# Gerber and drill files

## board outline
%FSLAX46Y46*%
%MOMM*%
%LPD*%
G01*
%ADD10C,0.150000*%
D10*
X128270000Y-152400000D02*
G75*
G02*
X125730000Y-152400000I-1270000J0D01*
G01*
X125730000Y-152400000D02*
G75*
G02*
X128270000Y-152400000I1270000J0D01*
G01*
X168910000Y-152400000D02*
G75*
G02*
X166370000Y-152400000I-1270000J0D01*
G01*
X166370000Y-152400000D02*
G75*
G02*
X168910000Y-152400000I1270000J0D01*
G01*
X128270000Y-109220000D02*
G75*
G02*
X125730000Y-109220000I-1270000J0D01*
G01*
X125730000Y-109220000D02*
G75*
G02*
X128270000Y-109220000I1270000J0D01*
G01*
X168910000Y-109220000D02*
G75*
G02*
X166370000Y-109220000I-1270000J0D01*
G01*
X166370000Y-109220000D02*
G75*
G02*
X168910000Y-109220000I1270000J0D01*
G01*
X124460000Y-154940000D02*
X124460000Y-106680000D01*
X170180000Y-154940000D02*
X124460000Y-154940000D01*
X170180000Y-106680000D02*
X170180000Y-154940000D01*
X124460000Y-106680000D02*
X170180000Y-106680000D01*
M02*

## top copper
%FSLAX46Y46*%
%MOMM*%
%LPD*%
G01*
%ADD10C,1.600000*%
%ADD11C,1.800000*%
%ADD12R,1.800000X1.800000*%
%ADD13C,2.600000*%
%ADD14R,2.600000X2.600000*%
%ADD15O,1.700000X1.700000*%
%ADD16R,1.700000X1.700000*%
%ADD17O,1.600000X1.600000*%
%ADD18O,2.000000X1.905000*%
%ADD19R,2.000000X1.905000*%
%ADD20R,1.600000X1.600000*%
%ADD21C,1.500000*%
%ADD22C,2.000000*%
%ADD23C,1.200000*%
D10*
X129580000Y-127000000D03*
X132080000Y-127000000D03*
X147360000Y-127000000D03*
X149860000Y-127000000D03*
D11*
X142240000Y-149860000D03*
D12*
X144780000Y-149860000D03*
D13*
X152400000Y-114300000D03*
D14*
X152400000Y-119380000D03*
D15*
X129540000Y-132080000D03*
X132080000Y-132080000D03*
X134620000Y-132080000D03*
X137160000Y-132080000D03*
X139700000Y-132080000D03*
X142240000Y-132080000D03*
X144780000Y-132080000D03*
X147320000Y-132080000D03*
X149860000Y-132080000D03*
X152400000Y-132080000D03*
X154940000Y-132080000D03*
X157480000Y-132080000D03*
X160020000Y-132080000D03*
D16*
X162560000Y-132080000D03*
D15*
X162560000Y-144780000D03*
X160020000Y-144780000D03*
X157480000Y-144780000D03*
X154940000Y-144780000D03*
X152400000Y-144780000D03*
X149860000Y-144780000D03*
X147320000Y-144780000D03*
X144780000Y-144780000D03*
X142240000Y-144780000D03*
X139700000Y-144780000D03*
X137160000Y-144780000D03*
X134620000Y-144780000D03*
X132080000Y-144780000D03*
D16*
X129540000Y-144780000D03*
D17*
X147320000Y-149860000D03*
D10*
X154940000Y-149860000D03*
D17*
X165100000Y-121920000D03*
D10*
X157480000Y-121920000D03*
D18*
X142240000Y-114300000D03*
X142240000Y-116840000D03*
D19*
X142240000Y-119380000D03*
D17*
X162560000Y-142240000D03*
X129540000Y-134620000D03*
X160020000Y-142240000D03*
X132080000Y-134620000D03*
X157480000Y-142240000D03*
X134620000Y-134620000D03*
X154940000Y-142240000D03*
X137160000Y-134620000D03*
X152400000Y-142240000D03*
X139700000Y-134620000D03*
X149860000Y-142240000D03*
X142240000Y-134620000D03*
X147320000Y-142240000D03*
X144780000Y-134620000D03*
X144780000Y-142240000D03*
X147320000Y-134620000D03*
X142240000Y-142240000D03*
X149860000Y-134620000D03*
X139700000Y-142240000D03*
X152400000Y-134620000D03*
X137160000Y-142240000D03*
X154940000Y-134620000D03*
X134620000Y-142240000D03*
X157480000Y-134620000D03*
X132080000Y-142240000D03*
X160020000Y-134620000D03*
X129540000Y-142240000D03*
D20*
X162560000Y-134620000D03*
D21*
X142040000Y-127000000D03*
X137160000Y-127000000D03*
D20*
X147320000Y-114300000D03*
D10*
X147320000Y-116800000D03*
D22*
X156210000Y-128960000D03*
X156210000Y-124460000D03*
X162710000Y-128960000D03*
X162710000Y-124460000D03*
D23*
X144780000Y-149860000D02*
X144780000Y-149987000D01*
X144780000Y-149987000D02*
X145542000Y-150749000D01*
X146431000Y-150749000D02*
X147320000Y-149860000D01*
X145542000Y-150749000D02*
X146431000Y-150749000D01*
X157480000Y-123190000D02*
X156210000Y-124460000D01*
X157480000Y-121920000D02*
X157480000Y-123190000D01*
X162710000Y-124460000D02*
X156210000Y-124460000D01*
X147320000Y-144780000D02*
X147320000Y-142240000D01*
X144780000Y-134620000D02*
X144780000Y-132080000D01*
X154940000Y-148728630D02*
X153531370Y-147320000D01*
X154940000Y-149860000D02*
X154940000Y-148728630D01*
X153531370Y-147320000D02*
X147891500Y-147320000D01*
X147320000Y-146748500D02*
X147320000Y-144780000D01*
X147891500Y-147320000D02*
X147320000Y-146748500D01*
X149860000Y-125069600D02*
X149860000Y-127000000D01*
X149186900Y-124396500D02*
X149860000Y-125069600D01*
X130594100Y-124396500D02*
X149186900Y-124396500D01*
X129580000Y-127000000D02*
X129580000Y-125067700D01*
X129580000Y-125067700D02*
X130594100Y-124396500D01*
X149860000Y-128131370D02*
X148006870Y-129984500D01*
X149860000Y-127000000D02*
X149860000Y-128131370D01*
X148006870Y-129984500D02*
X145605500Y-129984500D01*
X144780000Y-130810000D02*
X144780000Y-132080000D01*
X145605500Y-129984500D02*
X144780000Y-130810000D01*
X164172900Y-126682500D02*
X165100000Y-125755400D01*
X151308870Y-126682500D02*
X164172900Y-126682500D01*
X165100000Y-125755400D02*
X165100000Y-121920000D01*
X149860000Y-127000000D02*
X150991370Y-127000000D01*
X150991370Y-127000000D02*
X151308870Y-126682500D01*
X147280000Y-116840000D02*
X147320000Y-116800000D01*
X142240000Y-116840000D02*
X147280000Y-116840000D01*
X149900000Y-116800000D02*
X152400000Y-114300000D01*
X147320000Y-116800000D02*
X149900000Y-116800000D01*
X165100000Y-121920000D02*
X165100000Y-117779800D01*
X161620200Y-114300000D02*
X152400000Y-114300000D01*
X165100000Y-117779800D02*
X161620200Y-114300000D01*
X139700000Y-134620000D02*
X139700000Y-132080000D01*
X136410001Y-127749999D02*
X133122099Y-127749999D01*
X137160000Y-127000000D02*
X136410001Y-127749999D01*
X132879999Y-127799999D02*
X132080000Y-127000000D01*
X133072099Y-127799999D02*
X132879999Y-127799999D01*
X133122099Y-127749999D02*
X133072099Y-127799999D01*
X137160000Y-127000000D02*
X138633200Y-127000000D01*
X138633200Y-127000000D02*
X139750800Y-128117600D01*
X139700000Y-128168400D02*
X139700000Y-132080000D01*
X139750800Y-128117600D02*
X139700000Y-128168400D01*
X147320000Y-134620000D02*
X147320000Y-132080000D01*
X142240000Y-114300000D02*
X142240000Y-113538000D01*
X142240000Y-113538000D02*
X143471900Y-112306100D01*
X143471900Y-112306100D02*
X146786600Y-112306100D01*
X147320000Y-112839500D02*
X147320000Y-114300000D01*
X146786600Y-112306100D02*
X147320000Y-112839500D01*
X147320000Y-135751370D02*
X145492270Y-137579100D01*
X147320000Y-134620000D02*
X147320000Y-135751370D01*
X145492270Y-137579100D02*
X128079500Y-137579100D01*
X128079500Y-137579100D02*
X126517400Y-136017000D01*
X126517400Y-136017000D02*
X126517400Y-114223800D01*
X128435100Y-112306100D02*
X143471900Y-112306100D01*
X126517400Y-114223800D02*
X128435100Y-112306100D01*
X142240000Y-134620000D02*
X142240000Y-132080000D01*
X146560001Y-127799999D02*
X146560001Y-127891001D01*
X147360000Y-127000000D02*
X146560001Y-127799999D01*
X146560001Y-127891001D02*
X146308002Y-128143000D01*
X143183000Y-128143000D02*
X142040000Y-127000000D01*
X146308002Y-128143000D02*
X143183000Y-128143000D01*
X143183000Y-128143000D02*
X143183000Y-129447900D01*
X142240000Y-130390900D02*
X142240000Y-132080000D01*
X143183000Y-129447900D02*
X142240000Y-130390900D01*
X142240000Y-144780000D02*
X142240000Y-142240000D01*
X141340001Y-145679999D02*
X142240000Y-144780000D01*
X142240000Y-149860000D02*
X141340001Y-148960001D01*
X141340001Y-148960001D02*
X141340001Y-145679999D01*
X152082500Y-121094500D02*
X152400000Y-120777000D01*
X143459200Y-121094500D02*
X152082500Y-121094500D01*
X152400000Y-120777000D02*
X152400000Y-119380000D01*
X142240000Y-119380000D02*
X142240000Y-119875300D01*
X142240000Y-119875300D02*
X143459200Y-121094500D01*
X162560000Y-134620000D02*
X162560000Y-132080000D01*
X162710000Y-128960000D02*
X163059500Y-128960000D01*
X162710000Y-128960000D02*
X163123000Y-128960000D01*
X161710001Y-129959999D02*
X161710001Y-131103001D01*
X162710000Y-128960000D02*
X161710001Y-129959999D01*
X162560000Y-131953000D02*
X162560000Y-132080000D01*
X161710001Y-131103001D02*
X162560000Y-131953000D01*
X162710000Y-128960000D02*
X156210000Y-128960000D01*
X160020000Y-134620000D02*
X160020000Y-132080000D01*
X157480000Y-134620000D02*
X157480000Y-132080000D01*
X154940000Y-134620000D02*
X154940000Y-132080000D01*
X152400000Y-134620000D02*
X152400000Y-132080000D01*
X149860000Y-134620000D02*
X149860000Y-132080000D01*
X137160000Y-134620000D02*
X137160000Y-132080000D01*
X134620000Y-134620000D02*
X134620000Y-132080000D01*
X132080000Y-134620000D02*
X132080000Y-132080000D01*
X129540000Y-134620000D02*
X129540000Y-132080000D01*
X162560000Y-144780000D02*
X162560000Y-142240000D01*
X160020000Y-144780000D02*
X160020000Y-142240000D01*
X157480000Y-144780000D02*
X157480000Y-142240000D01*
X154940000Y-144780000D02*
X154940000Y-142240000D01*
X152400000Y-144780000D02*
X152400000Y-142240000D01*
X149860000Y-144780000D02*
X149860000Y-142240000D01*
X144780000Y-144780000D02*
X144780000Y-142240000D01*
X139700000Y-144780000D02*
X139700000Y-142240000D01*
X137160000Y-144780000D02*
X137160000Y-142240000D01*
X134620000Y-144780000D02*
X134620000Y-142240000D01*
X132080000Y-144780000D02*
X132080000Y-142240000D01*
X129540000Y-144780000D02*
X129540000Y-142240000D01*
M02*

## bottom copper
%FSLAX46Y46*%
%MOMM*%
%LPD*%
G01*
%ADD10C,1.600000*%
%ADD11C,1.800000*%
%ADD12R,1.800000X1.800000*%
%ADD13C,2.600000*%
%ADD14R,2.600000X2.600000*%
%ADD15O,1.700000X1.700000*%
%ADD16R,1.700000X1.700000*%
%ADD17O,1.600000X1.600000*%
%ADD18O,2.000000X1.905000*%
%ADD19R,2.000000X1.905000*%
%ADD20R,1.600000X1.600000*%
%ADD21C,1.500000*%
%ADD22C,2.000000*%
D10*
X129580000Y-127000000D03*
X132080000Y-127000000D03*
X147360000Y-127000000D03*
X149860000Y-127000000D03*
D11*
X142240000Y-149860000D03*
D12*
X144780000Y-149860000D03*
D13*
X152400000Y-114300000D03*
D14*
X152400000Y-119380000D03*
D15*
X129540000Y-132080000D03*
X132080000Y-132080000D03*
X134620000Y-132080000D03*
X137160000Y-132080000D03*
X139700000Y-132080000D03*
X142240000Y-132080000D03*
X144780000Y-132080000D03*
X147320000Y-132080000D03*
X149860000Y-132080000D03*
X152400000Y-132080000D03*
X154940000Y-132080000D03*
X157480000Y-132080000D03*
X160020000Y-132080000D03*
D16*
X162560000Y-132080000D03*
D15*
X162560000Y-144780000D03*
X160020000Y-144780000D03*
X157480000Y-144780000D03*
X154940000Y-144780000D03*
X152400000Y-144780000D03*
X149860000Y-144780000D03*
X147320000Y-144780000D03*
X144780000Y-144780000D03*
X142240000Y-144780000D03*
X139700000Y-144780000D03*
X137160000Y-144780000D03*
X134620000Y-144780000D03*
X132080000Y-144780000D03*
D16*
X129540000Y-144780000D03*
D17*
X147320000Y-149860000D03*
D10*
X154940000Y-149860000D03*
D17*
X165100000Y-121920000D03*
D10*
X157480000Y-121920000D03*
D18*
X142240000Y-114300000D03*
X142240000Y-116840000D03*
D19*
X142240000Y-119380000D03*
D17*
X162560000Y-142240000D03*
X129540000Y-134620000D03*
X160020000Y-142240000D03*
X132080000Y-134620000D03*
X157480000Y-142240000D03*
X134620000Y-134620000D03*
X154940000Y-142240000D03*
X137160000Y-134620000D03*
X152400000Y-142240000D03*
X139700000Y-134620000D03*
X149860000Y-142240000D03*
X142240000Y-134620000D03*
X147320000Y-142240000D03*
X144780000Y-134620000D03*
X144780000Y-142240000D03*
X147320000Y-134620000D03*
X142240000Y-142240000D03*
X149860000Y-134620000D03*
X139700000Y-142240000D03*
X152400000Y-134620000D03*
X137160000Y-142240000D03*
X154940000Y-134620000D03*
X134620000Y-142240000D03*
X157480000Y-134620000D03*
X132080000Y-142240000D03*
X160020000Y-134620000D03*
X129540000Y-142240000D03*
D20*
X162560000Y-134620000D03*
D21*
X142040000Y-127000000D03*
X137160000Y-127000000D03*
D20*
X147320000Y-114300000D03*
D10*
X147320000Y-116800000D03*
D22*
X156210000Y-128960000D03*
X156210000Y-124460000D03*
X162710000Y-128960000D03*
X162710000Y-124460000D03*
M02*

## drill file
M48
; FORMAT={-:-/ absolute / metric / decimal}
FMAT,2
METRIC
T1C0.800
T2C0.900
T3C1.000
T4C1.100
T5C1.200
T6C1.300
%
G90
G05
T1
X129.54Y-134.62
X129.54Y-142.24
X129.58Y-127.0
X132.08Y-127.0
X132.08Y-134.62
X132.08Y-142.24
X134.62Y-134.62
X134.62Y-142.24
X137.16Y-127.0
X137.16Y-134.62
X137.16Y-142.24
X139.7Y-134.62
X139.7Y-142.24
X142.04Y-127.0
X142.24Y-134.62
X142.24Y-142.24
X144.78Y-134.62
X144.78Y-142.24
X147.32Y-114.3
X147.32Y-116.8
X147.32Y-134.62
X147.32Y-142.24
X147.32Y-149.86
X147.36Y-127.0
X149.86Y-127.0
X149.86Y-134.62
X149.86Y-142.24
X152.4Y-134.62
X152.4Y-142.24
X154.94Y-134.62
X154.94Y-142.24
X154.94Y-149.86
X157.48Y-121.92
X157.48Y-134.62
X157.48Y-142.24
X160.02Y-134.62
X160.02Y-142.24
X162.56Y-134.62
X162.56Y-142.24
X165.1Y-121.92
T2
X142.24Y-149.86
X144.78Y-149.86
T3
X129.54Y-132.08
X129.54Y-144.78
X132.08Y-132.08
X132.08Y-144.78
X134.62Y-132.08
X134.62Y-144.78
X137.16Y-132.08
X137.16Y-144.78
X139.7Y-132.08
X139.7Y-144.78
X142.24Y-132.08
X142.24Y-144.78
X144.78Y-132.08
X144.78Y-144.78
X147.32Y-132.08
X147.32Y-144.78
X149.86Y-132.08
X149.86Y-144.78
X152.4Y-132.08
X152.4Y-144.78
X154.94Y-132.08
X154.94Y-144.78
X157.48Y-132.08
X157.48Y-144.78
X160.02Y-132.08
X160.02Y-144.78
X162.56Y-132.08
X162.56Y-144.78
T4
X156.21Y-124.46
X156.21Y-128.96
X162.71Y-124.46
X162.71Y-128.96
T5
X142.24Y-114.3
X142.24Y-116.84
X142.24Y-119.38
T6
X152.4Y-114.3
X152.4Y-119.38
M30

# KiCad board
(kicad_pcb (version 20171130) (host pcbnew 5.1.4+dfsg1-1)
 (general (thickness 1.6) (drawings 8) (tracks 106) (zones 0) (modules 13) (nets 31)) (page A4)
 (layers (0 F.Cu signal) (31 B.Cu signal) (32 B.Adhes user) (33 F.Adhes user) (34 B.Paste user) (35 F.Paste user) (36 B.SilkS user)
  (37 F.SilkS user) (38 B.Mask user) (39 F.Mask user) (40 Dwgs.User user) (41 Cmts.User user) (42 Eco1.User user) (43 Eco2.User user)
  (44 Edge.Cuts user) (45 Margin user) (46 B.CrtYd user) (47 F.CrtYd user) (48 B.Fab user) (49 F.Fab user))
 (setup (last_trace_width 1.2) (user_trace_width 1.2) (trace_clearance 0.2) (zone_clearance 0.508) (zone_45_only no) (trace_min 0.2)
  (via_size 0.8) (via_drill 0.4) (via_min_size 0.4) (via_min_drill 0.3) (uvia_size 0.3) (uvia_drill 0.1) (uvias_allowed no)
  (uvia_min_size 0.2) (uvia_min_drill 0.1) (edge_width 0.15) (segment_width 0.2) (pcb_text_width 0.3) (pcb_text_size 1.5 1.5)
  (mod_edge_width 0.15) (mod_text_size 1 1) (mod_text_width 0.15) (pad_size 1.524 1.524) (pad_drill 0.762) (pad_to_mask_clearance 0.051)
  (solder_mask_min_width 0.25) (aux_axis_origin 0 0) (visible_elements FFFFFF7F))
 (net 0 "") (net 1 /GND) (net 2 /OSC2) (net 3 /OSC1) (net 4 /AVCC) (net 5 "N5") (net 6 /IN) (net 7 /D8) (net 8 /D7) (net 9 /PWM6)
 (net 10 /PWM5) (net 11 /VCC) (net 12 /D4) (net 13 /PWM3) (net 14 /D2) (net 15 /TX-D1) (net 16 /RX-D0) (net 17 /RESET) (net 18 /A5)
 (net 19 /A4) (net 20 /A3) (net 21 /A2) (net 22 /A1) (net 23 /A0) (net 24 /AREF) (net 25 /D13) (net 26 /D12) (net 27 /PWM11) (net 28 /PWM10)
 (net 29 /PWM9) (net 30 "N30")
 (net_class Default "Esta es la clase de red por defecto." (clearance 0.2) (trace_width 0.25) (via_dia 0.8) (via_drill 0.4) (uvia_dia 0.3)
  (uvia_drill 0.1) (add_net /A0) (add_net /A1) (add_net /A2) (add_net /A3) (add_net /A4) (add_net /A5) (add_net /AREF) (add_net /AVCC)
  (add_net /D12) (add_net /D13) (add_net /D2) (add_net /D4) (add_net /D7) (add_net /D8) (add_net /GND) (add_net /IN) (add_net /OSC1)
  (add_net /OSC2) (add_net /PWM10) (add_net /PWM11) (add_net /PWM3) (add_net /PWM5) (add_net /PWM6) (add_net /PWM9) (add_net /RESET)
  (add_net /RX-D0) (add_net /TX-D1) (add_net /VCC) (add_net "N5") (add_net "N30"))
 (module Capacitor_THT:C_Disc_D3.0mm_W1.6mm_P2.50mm (layer F.Cu) (at 132.08 127 180)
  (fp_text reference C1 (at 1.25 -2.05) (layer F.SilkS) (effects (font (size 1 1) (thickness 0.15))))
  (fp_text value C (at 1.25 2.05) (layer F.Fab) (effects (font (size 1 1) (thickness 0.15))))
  (pad 2 thru_hole circle (at 2.5 0 180) (size 1.6 1.6) (drill 0.8) (layers *.Cu *.Mask) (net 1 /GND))
  (pad 1 thru_hole circle (at 0 0 180) (size 1.6 1.6) (drill 0.8) (layers *.Cu *.Mask) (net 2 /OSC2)))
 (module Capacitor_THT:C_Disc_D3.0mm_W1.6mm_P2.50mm (layer F.Cu) (at 149.86 127 180)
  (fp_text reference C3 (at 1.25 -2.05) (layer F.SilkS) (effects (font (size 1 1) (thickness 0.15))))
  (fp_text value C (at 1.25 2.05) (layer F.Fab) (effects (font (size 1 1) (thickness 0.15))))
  (pad 2 thru_hole circle (at 2.5 0 180) (size 1.6 1.6) (drill 0.8) (layers *.Cu *.Mask) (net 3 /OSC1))
  (pad 1 thru_hole circle (at 0 0 180) (size 1.6 1.6) (drill 0.8) (layers *.Cu *.Mask) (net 1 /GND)))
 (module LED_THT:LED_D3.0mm (layer F.Cu) (at 144.78 149.86 180)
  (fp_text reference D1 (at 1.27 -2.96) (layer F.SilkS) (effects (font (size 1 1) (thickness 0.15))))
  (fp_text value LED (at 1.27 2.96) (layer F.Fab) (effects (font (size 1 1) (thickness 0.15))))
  (pad 2 thru_hole circle (at 2.54 0 180) (size 1.8 1.8) (drill 0.9) (layers *.Cu *.Mask) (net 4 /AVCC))
  (pad 1 thru_hole rect (at 0 0 180) (size 1.8 1.8) (drill 0.9) (layers *.Cu *.Mask) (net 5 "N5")))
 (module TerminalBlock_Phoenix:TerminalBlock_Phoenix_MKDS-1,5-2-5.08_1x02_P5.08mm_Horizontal (layer F.Cu) (at 152.4 119.38 90)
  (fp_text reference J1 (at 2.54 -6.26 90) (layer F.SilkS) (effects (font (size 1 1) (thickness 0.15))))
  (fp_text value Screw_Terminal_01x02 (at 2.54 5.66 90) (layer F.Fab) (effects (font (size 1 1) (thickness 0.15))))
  (pad 2 thru_hole circle (at 5.08 0 90) (size 2.6 2.6) (drill 1.3) (layers *.Cu *.Mask) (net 1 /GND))
  (pad 1 thru_hole rect (at 0 0 90) (size 2.6 2.6) (drill 1.3) (layers *.Cu *.Mask) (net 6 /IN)))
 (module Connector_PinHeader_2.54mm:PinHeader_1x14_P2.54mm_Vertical (layer F.Cu) (at 162.56 132.08 270)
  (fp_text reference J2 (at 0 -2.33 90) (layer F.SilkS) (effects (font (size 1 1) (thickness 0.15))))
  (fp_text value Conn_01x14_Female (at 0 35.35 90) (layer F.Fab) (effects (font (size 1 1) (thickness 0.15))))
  (pad 14 thru_hole oval (at 0 33.02 270) (size 1.7 1.7) (drill 1) (layers *.Cu *.Mask) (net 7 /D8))
  (pad 13 thru_hole oval (at 0 30.48 270) (size 1.7 1.7) (drill 1) (layers *.Cu *.Mask) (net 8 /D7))
  (pad 12 thru_hole oval (at 0 27.94 270) (size 1.7 1.7) (drill 1) (layers *.Cu *.Mask) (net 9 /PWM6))
  (pad 11 thru_hole oval (at 0 25.4 270) (size 1.7 1.7) (drill 1) (layers *.Cu *.Mask) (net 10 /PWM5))
  (pad 10 thru_hole oval (at 0 22.86 270) (size 1.7 1.7) (drill 1) (layers *.Cu *.Mask) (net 2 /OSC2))
  (pad 9 thru_hole oval (at 0 20.32 270) (size 1.7 1.7) (drill 1) (layers *.Cu *.Mask) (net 3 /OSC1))
  (pad 8 thru_hole oval (at 0 17.78 270) (size 1.7 1.7) (drill 1) (layers *.Cu *.Mask) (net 1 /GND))
  (pad 7 thru_hole oval (at 0 15.24 270) (size 1.7 1.7) (drill 1) (layers *.Cu *.Mask) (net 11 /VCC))
  (pad 6 thru_hole oval (at 0 12.7 270) (size 1.7 1.7) (drill 1) (layers *.Cu *.Mask) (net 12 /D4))
  (pad 5 thru_hole oval (at 0 10.16 270) (size 1.7 1.7) (drill 1) (layers *.Cu *.Mask) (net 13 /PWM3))
  (pad 4 thru_hole oval (at 0 7.62 270) (size 1.7 1.7) (drill 1) (layers *.Cu *.Mask) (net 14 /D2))
  (pad 3 thru_hole oval (at 0 5.08 270) (size 1.7 1.7) (drill 1) (layers *.Cu *.Mask) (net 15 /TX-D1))
  (pad 2 thru_hole oval (at 0 2.54 270) (size 1.7 1.7) (drill 1) (layers *.Cu *.Mask) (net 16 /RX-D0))
  (pad 1 thru_hole rect (at 0 0 270) (size 1.7 1.7) (drill 1) (layers *.Cu *.Mask) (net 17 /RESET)))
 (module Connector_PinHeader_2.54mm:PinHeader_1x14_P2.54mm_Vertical (layer F.Cu) (at 129.54 144.78 90)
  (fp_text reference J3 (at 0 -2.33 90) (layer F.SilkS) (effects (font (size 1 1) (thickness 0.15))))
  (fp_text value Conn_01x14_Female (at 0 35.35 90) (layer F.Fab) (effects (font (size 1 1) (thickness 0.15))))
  (pad 14 thru_hole oval (at 0 33.02 90) (size 1.7 1.7) (drill 1) (layers *.Cu *.Mask) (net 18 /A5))
  (pad 13 thru_hole oval (at 0 30.48 90) (size 1.7 1.7) (drill 1) (layers *.Cu *.Mask) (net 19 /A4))
  (pad 12 thru_hole oval (at 0 27.94 90) (size 1.7 1.7) (drill 1) (layers *.Cu *.Mask) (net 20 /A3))
  (pad 11 thru_hole oval (at 0 25.4 90) (size 1.7 1.7) (drill 1) (layers *.Cu *.Mask) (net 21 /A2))
  (pad 10 thru_hole oval (at 0 22.86 90) (size 1.7 1.7) (drill 1) (layers *.Cu *.Mask) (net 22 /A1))
  (pad 9 thru_hole oval (at 0 20.32 90) (size 1.7 1.7) (drill 1) (layers *.Cu *.Mask) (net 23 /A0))
  (pad 8 thru_hole oval (at 0 17.78 90) (size 1.7 1.7) (drill 1) (layers *.Cu *.Mask) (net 1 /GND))
  (pad 7 thru_hole oval (at 0 15.24 90) (size 1.7 1.7) (drill 1) (layers *.Cu *.Mask) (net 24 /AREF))
  (pad 6 thru_hole oval (at 0 12.7 90) (size 1.7 1.7) (drill 1) (layers *.Cu *.Mask) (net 4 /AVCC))
  (pad 5 thru_hole oval (at 0 10.16 90) (size 1.7 1.7) (drill 1) (layers *.Cu *.Mask) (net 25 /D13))
  (pad 4 thru_hole oval (at 0 7.62 90) (size 1.7 1.7) (drill 1) (layers *.Cu *.Mask) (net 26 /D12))
  (pad 3 thru_hole oval (at 0 5.08 90) (size 1.7 1.7) (drill 1) (layers *.Cu *.Mask) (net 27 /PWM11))
  (pad 2 thru_hole oval (at 0 2.54 90) (size 1.7 1.7) (drill 1) (layers *.Cu *.Mask) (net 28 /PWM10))
  (pad 1 thru_hole rect (at 0 0 90) (size 1.7 1.7) (drill 1) (layers *.Cu *.Mask) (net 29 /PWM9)))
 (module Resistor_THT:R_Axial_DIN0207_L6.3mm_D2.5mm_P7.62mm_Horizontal (layer F.Cu) (at 154.94 149.86 180)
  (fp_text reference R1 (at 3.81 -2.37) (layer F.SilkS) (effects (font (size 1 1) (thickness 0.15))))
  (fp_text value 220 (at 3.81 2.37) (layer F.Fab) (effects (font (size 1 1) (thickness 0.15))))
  (pad 2 thru_hole oval (at 7.62 0 180) (size 1.6 1.6) (drill 0.8) (layers *.Cu *.Mask) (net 5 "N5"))
  (pad 1 thru_hole circle (at 0 0 180) (size 1.6 1.6) (drill 0.8) (layers *.Cu *.Mask) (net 1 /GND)))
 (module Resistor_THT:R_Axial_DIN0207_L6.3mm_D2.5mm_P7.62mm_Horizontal (layer F.Cu) (at 157.48 121.92)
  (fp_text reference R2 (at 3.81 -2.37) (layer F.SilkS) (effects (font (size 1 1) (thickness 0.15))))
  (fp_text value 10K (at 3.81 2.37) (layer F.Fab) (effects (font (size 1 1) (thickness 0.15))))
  (pad 2 thru_hole oval (at 7.62 0) (size 1.6 1.6) (drill 0.8) (layers *.Cu *.Mask) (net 1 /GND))
  (pad 1 thru_hole circle (at 0 0) (size 1.6 1.6) (drill 0.8) (layers *.Cu *.Mask) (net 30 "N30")))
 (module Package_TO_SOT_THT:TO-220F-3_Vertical (layer F.Cu) (at 142.24 119.38 90)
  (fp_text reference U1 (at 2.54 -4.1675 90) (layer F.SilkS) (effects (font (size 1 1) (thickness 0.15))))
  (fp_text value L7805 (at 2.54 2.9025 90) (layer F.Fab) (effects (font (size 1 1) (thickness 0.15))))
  (pad 3 thru_hole oval (at 5.08 0 90) (size 1.905 2) (drill 1.2) (layers *.Cu *.Mask) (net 11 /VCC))
  (pad 2 thru_hole oval (at 2.54 0 90) (size 1.905 2) (drill 1.2) (layers *.Cu *.Mask) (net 1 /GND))
  (pad 1 thru_hole rect (at 0 0 90) (size 1.905 2) (drill 1.2) (layers *.Cu *.Mask) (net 6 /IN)))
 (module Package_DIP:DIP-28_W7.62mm (layer F.Cu) (at 162.56 134.62 270)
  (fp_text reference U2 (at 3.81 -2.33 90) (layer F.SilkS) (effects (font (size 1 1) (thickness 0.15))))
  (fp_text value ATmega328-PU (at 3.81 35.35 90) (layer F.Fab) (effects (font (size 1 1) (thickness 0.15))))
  (pad 28 thru_hole oval (at 7.62 0 270) (size 1.6 1.6) (drill 0.8) (layers *.Cu *.Mask) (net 18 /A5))
  (pad 14 thru_hole oval (at 0 33.02 270) (size 1.6 1.6) (drill 0.8) (layers *.Cu *.Mask) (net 7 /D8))
  (pad 27 thru_hole oval (at 7.62 2.54 270) (size 1.6 1.6) (drill 0.8) (layers *.Cu *.Mask) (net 19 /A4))
  (pad 13 thru_hole oval (at 0 30.48 270) (size 1.6 1.6) (drill 0.8) (layers *.Cu *.Mask) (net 8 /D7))
  (pad 26 thru_hole oval (at 7.62 5.08 270) (size 1.6 1.6) (drill 0.8) (layers *.Cu *.Mask) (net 20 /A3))
  (pad 12 thru_hole oval (at 0 27.94 270) (size 1.6 1.6) (drill 0.8) (layers *.Cu *.Mask) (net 9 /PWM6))
  (pad 25 thru_hole oval (at 7.62 7.62 270) (size 1.6 1.6) (drill 0.8) (layers *.Cu *.Mask) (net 21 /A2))
  (pad 11 thru_hole oval (at 0 25.4 270) (size 1.6 1.6) (drill 0.8) (layers *.Cu *.Mask) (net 10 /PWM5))
  (pad 24 thru_hole oval (at 7.62 10.16 270) (size 1.6 1.6) (drill 0.8) (layers *.Cu *.Mask) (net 22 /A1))
  (pad 10 thru_hole oval (at 0 22.86 270) (size 1.6 1.6) (drill 0.8) (layers *.Cu *.Mask) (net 2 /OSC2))
  (pad 23 thru_hole oval (at 7.62 12.7 270) (size 1.6 1.6) (drill 0.8) (layers *.Cu *.Mask) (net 23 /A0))
  (pad 9 thru_hole oval (at 0 20.32 270) (size 1.6 1.6) (drill 0.8) (layers *.Cu *.Mask) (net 3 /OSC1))
  (pad 22 thru_hole oval (at 7.62 15.24 270) (size 1.6 1.6) (drill 0.8) (layers *.Cu *.Mask) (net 1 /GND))
  (pad 8 thru_hole oval (at 0 17.78 270) (size 1.6 1.6) (drill 0.8) (layers *.Cu *.Mask) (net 1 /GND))
  (pad 21 thru_hole oval (at 7.62 17.78 270) (size 1.6 1.6) (drill 0.8) (layers *.Cu *.Mask) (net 24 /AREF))
  (pad 7 thru_hole oval (at 0 15.24 270) (size 1.6 1.6) (drill 0.8) (layers *.Cu *.Mask) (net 11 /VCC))
  (pad 20 thru_hole oval (at 7.62 20.32 270) (size 1.6 1.6) (drill 0.8) (layers *.Cu *.Mask) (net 4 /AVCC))
  (pad 6 thru_hole oval (at 0 12.7 270) (size 1.6 1.6) (drill 0.8) (layers *.Cu *.Mask) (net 12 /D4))
  (pad 19 thru_hole oval (at 7.62 22.86 270) (size 1.6 1.6) (drill 0.8) (layers *.Cu *.Mask) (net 25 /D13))
  (pad 5 thru_hole oval (at 0 10.16 270) (size 1.6 1.6) (drill 0.8) (layers *.Cu *.Mask) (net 13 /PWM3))
  (pad 18 thru_hole oval (at 7.62 25.4 270) (size 1.6 1.6) (drill 0.8) (layers *.Cu *.Mask) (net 26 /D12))
  (pad 4 thru_hole oval (at 0 7.62 270) (size 1.6 1.6) (drill 0.8) (layers *.Cu *.Mask) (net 14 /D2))
  (pad 17 thru_hole oval (at 7.62 27.94 270) (size 1.6 1.6) (drill 0.8) (layers *.Cu *.Mask) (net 27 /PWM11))
  (pad 3 thru_hole oval (at 0 5.08 270) (size 1.6 1.6) (drill 0.8) (layers *.Cu *.Mask) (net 15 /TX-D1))
  (pad 16 thru_hole oval (at 7.62 30.48 270) (size 1.6 1.6) (drill 0.8) (layers *.Cu *.Mask) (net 28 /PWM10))
  (pad 2 thru_hole oval (at 0 2.54 270) (size 1.6 1.6) (drill 0.8) (layers *.Cu *.Mask) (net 16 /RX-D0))
  (pad 15 thru_hole oval (at 7.62 33.02 270) (size 1.6 1.6) (drill 0.8) (layers *.Cu *.Mask) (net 29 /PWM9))
  (pad 1 thru_hole rect (at 0 0 270) (size 1.6 1.6) (drill 0.8) (layers *.Cu *.Mask) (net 17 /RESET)))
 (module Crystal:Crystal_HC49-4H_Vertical (layer F.Cu) (at 137.16 127)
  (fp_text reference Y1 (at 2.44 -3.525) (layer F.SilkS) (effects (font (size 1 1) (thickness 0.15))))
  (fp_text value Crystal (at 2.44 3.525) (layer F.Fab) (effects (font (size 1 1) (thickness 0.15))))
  (pad 2 thru_hole circle (at 4.88 0) (size 1.5 1.5) (drill 0.8) (layers *.Cu *.Mask) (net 3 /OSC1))
  (pad 1 thru_hole circle (at 0 0) (size 1.5 1.5) (drill 0.8) (layers *.Cu *.Mask) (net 2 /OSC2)))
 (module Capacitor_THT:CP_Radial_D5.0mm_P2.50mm (layer F.Cu) (at 147.32 114.3 270)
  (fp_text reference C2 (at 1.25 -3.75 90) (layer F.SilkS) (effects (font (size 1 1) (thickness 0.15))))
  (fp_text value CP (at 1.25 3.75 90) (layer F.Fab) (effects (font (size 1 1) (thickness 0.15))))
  (pad 1 thru_hole rect (at 0 0 270) (size 1.6 1.6) (drill 0.8) (layers *.Cu *.Mask) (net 11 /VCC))
  (pad 2 thru_hole circle (at 2.5 0 270) (size 1.6 1.6) (drill 0.8) (layers *.Cu *.Mask) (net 1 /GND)))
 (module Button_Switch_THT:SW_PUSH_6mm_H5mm (layer F.Cu) (at 156.21 124.46)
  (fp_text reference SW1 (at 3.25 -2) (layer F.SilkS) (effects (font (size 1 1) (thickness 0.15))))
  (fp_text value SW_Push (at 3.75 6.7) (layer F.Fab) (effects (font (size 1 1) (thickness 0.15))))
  (pad 2 thru_hole circle (at 0 4.5 90) (size 2 2) (drill 1.1) (layers *.Cu *.Mask) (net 17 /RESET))
  (pad 1 thru_hole circle (at 0 0 90) (size 2 2) (drill 1.1) (layers *.Cu *.Mask) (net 30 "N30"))
  (pad 2 thru_hole circle (at 6.5 4.5 90) (size 2 2) (drill 1.1) (layers *.Cu *.Mask) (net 17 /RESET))
  (pad 1 thru_hole circle (at 6.5 0 90) (size 2 2) (drill 1.1) (layers *.Cu *.Mask) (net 30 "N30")))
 (gr_circle (center 127 152.4) (end 127 153.67) (layer Edge.Cuts) (width 0.15))
 (gr_circle (center 167.64 152.4) (end 167.64 151.13) (layer Edge.Cuts) (width 0.15))
 (gr_circle (center 127 109.22) (end 127 107.95) (layer Edge.Cuts) (width 0.15))
 (gr_circle (center 167.64 109.22) (end 167.64 110.49) (layer Edge.Cuts) (width 0.15))
 (gr_line (start 124.46 154.94) (end 124.46 106.68) (layer Edge.Cuts) (width 0.15))
 (gr_line (start 170.18 154.94) (end 124.46 154.94) (layer Edge.Cuts) (width 0.15))
 (gr_line (start 170.18 106.68) (end 170.18 154.94) (layer Edge.Cuts) (width 0.15))
 (gr_line (start 124.46 106.68) (end 170.18 106.68) (layer Edge.Cuts) (width 0.15))
 (segment (start 144.78 149.86) (end 144.78 149.987) (width 1.2) (layer F.Cu) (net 5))
 (segment (start 144.78 149.987) (end 145.542 150.749) (width 1.2) (layer F.Cu) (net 5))
 (segment (start 146.431 150.749) (end 147.32 149.86) (width 1.2) (layer F.Cu) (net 5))
 (segment (start 145.542 150.749) (end 146.431 150.749) (width 1.2) (layer F.Cu) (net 5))
 (segment (start 157.48 123.19) (end 156.21 124.46) (width 1.2) (layer F.Cu) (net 30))
 (segment (start 157.48 121.92) (end 157.48 123.19) (width 1.2) (layer F.Cu) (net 30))
 (segment (start 162.71 124.46) (end 156.21 124.46) (width 1.2) (layer F.Cu) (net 30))
 (segment (start 147.32 144.78) (end 147.32 142.24) (width 1.2) (layer F.Cu) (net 1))
 (segment (start 144.78 134.62) (end 144.78 132.08) (width 1.2) (layer F.Cu) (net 1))
 (segment (start 154.94 148.72863) (end 153.53137 147.32) (width 1.2) (layer F.Cu) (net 1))
 (segment (start 154.94 149.86) (end 154.94 148.72863) (width 1.2) (layer F.Cu) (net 1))
 (segment (start 153.53137 147.32) (end 147.8915 147.32) (width 1.2) (layer F.Cu) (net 1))
 (segment (start 147.32 146.7485) (end 147.32 144.78) (width 1.2) (layer F.Cu) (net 1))
 (segment (start 147.8915 147.32) (end 147.32 146.7485) (width 1.2) (layer F.Cu) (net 1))
 (segment (start 149.86 125.0696) (end 149.86 127) (width 1.2) (layer F.Cu) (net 1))
 (segment (start 149.1869 124.3965) (end 149.86 125.0696) (width 1.2) (layer F.Cu) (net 1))
 (segment (start 130.5941 124.3965) (end 149.1869 124.3965) (width 1.2) (layer F.Cu) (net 1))
 (segment (start 129.58 127) (end 129.58 125.0677) (width 1.2) (layer F.Cu) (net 1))
 (segment (start 129.58 125.0677) (end 130.5941 124.3965) (width 1.2) (layer F.Cu) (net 1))
 (segment (start 149.86 128.13137) (end 148.00687 129.9845) (width 1.2) (layer F.Cu) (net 1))
 (segment (start 149.86 127) (end 149.86 128.13137) (width 1.2) (layer F.Cu) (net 1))
 (segment (start 148.00687 129.9845) (end 145.6055 129.9845) (width 1.2) (layer F.Cu) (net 1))
 (segment (start 144.78 130.81) (end 144.78 132.08) (width 1.2) (layer F.Cu) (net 1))
 (segment (start 145.6055 129.9845) (end 144.78 130.81) (width 1.2) (layer F.Cu) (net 1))
 (segment (start 164.1729 126.6825) (end 165.1 125.7554) (width 1.2) (layer F.Cu) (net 1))
 (segment (start 151.30887 126.6825) (end 164.1729 126.6825) (width 1.2) (layer F.Cu) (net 1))
 (segment (start 165.1 125.7554) (end 165.1 121.92) (width 1.2) (layer F.Cu) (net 1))
 (segment (start 149.86 127) (end 150.99137 127) (width 1.2) (layer F.Cu) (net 1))
 (segment (start 150.99137 127) (end 151.30887 126.6825) (width 1.2) (layer F.Cu) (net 1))
 (segment (start 147.28 116.84) (end 147.32 116.8) (width 1.2) (layer F.Cu) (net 1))
 (segment (start 142.24 116.84) (end 147.28 116.84) (width 1.2) (layer F.Cu) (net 1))
 (segment (start 149.9 116.8) (end 152.4 114.3) (width 1.2) (layer F.Cu) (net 1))
 (segment (start 147.32 116.8) (end 149.9 116.8) (width 1.2) (layer F.Cu) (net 1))
 (segment (start 165.1 121.92) (end 165.1 117.7798) (width 1.2) (layer F.Cu) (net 1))
 (segment (start 161.6202 114.3) (end 152.4 114.3) (width 1.2) (layer F.Cu) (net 1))
 (segment (start 165.1 117.7798) (end 161.6202 114.3) (width 1.2) (layer F.Cu) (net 1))
 (segment (start 139.7 134.62) (end 139.7 132.08) (width 1.2) (layer F.Cu) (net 2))
 (segment (start 136.410001 127.749999) (end 133.122099 127.749999) (width 1.2) (layer F.Cu) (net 2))
 (segment (start 137.16 127) (end 136.410001 127.749999) (width 1.2) (layer F.Cu) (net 2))
 (segment (start 132.879999 127.799999) (end 132.08 127) (width 1.2) (layer F.Cu) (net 2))
 (segment (start 133.072099 127.799999) (end 132.879999 127.799999) (width 1.2) (layer F.Cu) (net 2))
 (segment (start 133.122099 127.749999) (end 133.072099 127.799999) (width 1.2) (layer F.Cu) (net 2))
 (segment (start 137.16 127) (end 138.6332 127) (width 1.2) (layer F.Cu) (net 2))
 (segment (start 138.6332 127) (end 139.7508 128.1176) (width 1.2) (layer F.Cu) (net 2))
 (segment (start 139.7 128.1684) (end 139.7 132.08) (width 1.2) (layer F.Cu) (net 2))
 (segment (start 139.7508 128.1176) (end 139.7 128.1684) (width 1.2) (layer F.Cu) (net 2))
 (segment (start 147.32 134.62) (end 147.32 132.08) (width 1.2) (layer F.Cu) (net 11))
 (segment (start 142.24 114.3) (end 142.24 113.538) (width 1.2) (layer F.Cu) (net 11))
 (segment (start 142.24 113.538) (end 143.4719 112.3061) (width 1.2) (layer F.Cu) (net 11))
 (segment (start 143.4719 112.3061) (end 146.7866 112.3061) (width 1.2) (layer F.Cu) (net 11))
 (segment (start 147.32 112.8395) (end 147.32 114.3) (width 1.2) (layer F.Cu) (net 11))
 (segment (start 146.7866 112.3061) (end 147.32 112.8395) (width 1.2) (layer F.Cu) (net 11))
 (segment (start 147.32 135.75137) (end 145.49227 137.5791) (width 1.2) (layer F.Cu) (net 11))
 (segment (start 147.32 134.62) (end 147.32 135.75137) (width 1.2) (layer F.Cu) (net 11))
 (segment (start 145.49227 137.5791) (end 128.0795 137.5791) (width 1.2) (layer F.Cu) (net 11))
 (segment (start 128.0795 137.5791) (end 126.5174 136.017) (width 1.2) (layer F.Cu) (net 11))
 (segment (start 126.5174 136.017) (end 126.5174 114.2238) (width 1.2) (layer F.Cu) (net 11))
 (segment (start 128.4351 112.3061) (end 143.4719 112.3061) (width 1.2) (layer F.Cu) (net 11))
 (segment (start 126.5174 114.2238) (end 128.4351 112.3061) (width 1.2) (layer F.Cu) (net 11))
 (segment (start 142.24 134.62) (end 142.24 132.08) (width 1.2) (layer F.Cu) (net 3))
 (segment (start 146.560001 127.799999) (end 146.560001 127.891001) (width 1.2) (layer F.Cu) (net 3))
 (segment (start 147.36 127) (end 146.560001 127.799999) (width 1.2) (layer F.Cu) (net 3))
 (segment (start 146.560001 127.891001) (end 146.308002 128.143) (width 1.2) (layer F.Cu) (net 3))
 (segment (start 143.183 128.143) (end 142.04 127) (width 1.2) (layer F.Cu) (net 3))
 (segment (start 146.308002 128.143) (end 143.183 128.143) (width 1.2) (layer F.Cu) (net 3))
 (segment (start 143.183 128.143) (end 143.183 129.4479) (width 1.2) (layer F.Cu) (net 3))
 (segment (start 142.24 130.3909) (end 142.24 132.08) (width 1.2) (layer F.Cu) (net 3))
 (segment (start 143.183 129.4479) (end 142.24 130.3909) (width 1.2) (layer F.Cu) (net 3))
 (segment (start 142.24 144.78) (end 142.24 142.24) (width 1.2) (layer F.Cu) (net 4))
 (segment (start 141.340001 145.679999) (end 142.24 144.78) (width 1.2) (layer F.Cu) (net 4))
 (segment (start 142.24 149.86) (end 141.340001 148.960001) (width 1.2) (layer F.Cu) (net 4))
 (segment (start 141.340001 148.960001) (end 141.340001 145.679999) (width 1.2) (layer F.Cu) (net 4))
 (segment (start 152.0825 121.0945) (end 152.4 120.777) (width 1.2) (layer F.Cu) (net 6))
 (segment (start 143.4592 121.0945) (end 152.0825 121.0945) (width 1.2) (layer F.Cu) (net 6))
 (segment (start 152.4 120.777) (end 152.4 119.38) (width 1.2) (layer F.Cu) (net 6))
 (segment (start 142.24 119.38) (end 142.24 119.8753) (width 1.2) (layer F.Cu) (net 6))
 (segment (start 142.24 119.8753) (end 143.4592 121.0945) (width 1.2) (layer F.Cu) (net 6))
 (segment (start 162.56 134.62) (end 162.56 132.08) (width 1.2) (layer F.Cu) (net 17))
 (segment (start 162.71 128.96) (end 163.0595 128.96) (width 1.2) (layer F.Cu) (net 17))
 (segment (start 162.71 128.96) (end 163.123 128.96) (width 1.2) (layer F.Cu) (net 17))
 (segment (start 161.710001 129.959999) (end 161.710001 131.103001) (width 1.2) (layer F.Cu) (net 17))
 (segment (start 162.71 128.96) (end 161.710001 129.959999) (width 1.2) (layer F.Cu) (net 17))
 (segment (start 162.56 131.953) (end 162.56 132.08) (width 1.2) (layer F.Cu) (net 17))
 (segment (start 161.710001 131.103001) (end 162.56 131.953) (width 1.2) (layer F.Cu) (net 17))
 (segment (start 162.71 128.96) (end 156.21 128.96) (width 1.2) (layer F.Cu) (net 17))
 (segment (start 160.02 134.62) (end 160.02 132.08) (width 1.2) (layer F.Cu) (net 16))
 (segment (start 157.48 134.62) (end 157.48 132.08) (width 1.2) (layer F.Cu) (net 15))
 (segment (start 154.94 134.62) (end 154.94 132.08) (width 1.2) (layer F.Cu) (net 14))
 (segment (start 152.4 134.62) (end 152.4 132.08) (width 1.2) (layer F.Cu) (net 13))
 (segment (start 149.86 134.62) (end 149.86 132.08) (width 1.2) (layer F.Cu) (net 12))
 (segment (start 137.16 134.62) (end 137.16 132.08) (width 1.2) (layer F.Cu) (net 10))
 (segment (start 134.62 134.62) (end 134.62 132.08) (width 1.2) (layer F.Cu) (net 9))
 (segment (start 132.08 134.62) (end 132.08 132.08) (width 1.2) (layer F.Cu) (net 8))
 (segment (start 129.54 134.62) (end 129.54 132.08) (width 1.2) (layer F.Cu) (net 7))
 (segment (start 162.56 144.78) (end 162.56 142.24) (width 1.2) (layer F.Cu) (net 18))
 (segment (start 160.02 144.78) (end 160.02 142.24) (width 1.2) (layer F.Cu) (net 19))
 (segment (start 157.48 144.78) (end 157.48 142.24) (width 1.2) (layer F.Cu) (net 20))
 (segment (start 154.94 144.78) (end 154.94 142.24) (width 1.2) (layer F.Cu) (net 21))
 (segment (start 152.4 144.78) (end 152.4 142.24) (width 1.2) (layer F.Cu) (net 22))
 (segment (start 149.86 144.78) (end 149.86 142.24) (width 1.2) (layer F.Cu) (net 23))
 (segment (start 144.78 144.78) (end 144.78 142.24) (width 1.2) (layer F.Cu) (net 24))
 (segment (start 139.7 144.78) (end 139.7 142.24) (width 1.2) (layer F.Cu) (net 25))
 (segment (start 137.16 144.78) (end 137.16 142.24) (width 1.2) (layer F.Cu) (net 26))
 (segment (start 134.62 144.78) (end 134.62 142.24) (width 1.2) (layer F.Cu) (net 27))
 (segment (start 132.08 144.78) (end 132.08 142.24) (width 1.2) (layer F.Cu) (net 28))
 (segment (start 129.54 144.78) (end 129.54 142.24) (width 1.2) (layer F.Cu) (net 29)))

